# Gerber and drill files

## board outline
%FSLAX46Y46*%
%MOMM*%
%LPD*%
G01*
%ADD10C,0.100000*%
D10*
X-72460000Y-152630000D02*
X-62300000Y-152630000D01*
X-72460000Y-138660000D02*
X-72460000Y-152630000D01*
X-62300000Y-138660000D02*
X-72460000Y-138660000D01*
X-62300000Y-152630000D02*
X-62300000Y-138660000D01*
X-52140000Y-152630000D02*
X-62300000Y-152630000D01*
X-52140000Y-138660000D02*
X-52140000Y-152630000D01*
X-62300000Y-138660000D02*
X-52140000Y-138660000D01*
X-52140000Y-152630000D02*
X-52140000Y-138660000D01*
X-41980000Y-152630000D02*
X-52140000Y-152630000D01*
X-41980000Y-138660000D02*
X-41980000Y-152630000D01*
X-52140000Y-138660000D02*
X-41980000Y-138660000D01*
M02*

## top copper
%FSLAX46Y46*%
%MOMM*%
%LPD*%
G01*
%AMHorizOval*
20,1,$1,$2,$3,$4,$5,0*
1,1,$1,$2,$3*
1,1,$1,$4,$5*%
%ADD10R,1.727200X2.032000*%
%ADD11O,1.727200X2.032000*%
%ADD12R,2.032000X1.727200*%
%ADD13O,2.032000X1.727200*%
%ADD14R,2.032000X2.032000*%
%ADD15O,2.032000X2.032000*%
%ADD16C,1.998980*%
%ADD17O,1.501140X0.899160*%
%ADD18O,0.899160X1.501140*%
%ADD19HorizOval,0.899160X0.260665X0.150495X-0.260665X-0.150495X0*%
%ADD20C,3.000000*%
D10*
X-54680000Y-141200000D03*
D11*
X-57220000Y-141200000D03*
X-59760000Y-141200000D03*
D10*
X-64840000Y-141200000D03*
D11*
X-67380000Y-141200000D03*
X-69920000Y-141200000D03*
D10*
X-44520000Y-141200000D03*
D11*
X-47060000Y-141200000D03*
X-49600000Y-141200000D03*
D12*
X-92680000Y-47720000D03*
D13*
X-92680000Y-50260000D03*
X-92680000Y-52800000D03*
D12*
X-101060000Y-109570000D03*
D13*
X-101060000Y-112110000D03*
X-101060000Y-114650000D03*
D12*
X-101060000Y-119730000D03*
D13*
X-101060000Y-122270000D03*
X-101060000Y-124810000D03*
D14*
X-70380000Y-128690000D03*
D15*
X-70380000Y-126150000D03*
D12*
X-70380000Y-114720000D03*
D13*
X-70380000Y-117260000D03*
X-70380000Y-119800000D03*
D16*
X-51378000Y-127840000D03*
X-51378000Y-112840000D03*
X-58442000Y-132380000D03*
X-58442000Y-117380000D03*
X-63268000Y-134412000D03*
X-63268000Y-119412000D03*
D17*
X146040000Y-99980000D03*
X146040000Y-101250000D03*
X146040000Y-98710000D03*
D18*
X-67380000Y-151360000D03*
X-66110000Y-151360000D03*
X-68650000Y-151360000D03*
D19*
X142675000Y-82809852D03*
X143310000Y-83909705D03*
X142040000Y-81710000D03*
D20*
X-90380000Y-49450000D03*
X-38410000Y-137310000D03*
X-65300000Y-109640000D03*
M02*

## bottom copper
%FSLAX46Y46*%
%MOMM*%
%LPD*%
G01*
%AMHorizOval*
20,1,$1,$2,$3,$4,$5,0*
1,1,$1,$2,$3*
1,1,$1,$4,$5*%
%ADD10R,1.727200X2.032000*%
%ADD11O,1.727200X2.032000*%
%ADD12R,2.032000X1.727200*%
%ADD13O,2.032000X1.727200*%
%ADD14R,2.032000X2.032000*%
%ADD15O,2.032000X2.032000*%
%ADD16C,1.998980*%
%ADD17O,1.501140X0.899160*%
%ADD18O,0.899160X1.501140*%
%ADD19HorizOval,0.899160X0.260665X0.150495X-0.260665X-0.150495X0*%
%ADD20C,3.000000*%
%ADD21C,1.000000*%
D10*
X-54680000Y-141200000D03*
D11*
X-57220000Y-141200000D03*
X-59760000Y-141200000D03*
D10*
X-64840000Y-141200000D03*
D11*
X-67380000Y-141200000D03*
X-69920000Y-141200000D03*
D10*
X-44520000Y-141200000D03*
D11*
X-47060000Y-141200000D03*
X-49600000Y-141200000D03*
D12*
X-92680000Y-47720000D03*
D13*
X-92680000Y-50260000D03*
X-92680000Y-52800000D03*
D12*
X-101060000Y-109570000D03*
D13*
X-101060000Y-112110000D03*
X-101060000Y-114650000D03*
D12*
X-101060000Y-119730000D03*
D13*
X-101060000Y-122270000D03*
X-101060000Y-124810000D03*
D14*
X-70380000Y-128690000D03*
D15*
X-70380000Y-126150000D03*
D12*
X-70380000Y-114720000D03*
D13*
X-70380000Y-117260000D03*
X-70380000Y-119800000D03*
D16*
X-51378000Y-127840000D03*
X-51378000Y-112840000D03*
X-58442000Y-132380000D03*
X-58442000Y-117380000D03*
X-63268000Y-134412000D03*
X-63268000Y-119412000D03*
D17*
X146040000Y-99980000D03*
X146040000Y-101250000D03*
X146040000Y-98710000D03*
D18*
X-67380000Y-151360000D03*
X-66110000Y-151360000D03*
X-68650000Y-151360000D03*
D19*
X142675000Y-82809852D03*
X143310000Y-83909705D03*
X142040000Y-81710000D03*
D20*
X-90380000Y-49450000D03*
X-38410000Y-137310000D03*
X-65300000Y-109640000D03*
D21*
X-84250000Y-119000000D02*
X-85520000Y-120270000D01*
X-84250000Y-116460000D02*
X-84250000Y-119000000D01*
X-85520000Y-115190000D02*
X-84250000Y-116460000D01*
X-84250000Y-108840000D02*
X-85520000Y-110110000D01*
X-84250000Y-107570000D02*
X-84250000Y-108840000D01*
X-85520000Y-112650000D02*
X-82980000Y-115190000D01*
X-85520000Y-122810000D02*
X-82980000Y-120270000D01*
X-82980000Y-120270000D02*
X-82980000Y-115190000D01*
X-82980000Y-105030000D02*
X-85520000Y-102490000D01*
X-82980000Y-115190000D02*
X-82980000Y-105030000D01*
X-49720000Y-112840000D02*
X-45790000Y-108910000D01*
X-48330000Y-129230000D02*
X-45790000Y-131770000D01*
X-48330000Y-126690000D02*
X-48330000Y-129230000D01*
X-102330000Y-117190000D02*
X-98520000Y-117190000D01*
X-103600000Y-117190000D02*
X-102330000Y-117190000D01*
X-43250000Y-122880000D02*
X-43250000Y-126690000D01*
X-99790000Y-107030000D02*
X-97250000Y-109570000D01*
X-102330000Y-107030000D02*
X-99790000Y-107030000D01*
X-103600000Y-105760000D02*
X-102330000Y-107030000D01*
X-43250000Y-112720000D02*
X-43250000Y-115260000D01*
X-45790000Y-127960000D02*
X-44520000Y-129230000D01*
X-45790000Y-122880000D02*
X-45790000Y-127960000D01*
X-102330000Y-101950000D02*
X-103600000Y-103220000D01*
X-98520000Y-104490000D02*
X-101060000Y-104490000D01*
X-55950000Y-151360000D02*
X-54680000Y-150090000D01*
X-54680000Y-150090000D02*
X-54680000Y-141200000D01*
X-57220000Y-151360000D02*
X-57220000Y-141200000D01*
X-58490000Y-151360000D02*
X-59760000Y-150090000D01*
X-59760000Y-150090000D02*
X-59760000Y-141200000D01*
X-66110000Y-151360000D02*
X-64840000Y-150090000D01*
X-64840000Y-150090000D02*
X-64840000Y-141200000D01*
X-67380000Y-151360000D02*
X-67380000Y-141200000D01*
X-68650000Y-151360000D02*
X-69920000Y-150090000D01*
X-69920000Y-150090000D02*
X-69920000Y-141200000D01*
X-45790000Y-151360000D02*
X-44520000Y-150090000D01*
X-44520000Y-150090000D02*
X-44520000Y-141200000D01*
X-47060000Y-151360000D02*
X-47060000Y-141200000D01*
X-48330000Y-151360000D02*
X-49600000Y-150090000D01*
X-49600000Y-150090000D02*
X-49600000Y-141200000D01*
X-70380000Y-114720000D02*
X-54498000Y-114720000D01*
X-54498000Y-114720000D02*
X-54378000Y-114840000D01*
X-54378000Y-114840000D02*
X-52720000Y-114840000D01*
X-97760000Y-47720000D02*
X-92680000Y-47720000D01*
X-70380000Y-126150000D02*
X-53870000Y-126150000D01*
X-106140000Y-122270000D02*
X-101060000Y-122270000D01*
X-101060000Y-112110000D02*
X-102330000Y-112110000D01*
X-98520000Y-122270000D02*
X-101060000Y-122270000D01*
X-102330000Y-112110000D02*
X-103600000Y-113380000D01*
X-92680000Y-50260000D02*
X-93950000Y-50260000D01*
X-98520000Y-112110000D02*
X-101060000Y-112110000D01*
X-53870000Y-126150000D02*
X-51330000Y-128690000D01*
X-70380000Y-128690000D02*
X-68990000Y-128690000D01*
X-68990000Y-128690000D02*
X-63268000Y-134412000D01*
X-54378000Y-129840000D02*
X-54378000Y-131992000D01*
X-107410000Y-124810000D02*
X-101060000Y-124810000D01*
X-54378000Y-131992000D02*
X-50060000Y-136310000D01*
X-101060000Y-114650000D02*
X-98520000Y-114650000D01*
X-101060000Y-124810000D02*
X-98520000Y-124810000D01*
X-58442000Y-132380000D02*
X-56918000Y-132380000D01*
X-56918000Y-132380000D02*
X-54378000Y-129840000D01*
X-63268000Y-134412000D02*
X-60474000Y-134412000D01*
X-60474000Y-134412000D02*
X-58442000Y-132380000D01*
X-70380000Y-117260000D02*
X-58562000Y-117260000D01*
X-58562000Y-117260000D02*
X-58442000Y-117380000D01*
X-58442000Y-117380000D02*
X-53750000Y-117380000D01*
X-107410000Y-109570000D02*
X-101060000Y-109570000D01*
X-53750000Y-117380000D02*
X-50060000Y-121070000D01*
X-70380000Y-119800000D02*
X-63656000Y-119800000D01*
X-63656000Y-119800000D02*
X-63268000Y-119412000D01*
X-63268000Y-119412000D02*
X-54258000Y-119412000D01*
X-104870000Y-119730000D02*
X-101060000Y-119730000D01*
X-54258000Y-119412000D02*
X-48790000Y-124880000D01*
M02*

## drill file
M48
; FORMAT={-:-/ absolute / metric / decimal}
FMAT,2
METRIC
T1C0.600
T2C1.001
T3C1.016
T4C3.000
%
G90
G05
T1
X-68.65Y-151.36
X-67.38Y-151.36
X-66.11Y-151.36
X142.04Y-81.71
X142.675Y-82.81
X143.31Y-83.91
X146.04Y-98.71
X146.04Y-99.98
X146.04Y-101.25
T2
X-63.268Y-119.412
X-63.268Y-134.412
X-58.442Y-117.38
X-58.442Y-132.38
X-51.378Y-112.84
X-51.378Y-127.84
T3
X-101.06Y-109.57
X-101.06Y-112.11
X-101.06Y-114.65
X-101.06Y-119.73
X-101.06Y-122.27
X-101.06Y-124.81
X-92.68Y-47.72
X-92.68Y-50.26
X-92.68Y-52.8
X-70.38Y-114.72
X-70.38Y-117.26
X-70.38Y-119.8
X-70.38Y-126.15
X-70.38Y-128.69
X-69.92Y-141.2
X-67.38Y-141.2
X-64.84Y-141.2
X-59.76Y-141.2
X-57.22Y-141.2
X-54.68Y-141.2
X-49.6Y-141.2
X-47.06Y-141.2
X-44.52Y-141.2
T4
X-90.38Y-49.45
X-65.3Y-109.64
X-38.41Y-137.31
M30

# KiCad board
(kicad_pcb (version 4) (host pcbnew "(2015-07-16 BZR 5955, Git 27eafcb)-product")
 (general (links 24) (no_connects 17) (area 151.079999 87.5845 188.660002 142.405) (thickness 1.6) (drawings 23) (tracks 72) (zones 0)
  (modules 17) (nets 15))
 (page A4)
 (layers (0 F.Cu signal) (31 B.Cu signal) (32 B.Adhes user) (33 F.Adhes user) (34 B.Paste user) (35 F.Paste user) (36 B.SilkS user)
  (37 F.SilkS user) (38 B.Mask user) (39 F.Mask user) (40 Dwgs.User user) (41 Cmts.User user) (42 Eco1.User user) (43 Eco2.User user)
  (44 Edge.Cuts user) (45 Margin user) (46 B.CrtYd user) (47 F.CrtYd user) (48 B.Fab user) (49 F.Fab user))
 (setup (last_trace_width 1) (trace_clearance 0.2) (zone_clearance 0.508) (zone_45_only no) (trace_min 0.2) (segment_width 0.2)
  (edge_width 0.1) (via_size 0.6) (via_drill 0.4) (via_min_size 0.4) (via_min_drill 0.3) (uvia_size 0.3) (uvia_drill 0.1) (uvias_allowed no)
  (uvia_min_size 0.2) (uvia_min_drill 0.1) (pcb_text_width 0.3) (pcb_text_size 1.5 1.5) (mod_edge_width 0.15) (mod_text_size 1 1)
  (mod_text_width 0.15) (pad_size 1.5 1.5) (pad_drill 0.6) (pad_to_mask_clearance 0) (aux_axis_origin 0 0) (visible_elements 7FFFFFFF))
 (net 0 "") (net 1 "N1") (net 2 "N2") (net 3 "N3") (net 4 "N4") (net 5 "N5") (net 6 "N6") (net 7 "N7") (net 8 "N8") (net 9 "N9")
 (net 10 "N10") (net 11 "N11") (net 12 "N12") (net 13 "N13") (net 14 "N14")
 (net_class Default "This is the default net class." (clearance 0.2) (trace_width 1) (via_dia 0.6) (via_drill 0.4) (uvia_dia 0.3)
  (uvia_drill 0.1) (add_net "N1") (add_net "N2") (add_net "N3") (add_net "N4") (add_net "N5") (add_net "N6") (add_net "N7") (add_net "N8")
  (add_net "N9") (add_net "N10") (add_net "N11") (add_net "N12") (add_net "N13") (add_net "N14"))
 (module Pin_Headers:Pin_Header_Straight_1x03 (layer F.Cu) (at -54.68 141.2 270)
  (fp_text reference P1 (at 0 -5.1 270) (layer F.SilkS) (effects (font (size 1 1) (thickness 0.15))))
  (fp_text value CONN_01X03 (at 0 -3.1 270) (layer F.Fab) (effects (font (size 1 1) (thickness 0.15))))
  (pad 1 thru_hole rect (at 0 0 270) (size 2.032 1.7272) (drill 1.016) (layers *.Cu *.Mask F.SilkS) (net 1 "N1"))
  (pad 2 thru_hole oval (at 0 2.54 270) (size 2.032 1.7272) (drill 1.016) (layers *.Cu *.Mask F.SilkS) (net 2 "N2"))
  (pad 3 thru_hole oval (at 0 5.08 270) (size 2.032 1.7272) (drill 1.016) (layers *.Cu *.Mask F.SilkS) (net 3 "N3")))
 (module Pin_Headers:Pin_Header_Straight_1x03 (layer F.Cu) (at -64.84 141.2 270)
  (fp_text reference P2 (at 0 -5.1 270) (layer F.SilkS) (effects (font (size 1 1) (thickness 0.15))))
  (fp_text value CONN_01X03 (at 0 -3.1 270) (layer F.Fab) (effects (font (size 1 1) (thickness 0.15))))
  (pad 1 thru_hole rect (at 0 0 270) (size 2.032 1.7272) (drill 1.016) (layers *.Cu *.Mask F.SilkS) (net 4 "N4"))
  (pad 2 thru_hole oval (at 0 2.54 270) (size 2.032 1.7272) (drill 1.016) (layers *.Cu *.Mask F.SilkS) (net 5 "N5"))
  (pad 3 thru_hole oval (at 0 5.08 270) (size 2.032 1.7272) (drill 1.016) (layers *.Cu *.Mask F.SilkS) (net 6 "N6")))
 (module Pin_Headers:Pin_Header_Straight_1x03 (layer F.Cu) (at -44.52 141.2 270)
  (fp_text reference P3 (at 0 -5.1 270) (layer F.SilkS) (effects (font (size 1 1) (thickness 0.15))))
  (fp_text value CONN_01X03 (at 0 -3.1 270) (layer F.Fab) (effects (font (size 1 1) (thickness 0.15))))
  (pad 1 thru_hole rect (at 0 0 270) (size 2.032 1.7272) (drill 1.016) (layers *.Cu *.Mask F.SilkS) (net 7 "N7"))
  (pad 2 thru_hole oval (at 0 2.54 270) (size 2.032 1.7272) (drill 1.016) (layers *.Cu *.Mask F.SilkS) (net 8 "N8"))
  (pad 3 thru_hole oval (at 0 5.08 270) (size 2.032 1.7272) (drill 1.016) (layers *.Cu *.Mask F.SilkS) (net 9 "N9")))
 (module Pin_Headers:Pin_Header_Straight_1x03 (layer F.Cu) (at -92.68 47.72)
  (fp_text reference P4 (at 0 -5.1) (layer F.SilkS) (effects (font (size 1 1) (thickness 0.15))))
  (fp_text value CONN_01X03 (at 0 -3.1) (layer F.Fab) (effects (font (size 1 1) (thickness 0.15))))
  (pad 1 thru_hole rect (at 0 0) (size 2.032 1.7272) (drill 1.016) (layers *.Cu *.Mask F.SilkS) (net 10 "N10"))
  (pad 2 thru_hole oval (at 0 2.54) (size 2.032 1.7272) (drill 1.016) (layers *.Cu *.Mask F.SilkS) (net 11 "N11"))
  (pad 3 thru_hole oval (at 0 5.08) (size 2.032 1.7272) (drill 1.016) (layers *.Cu *.Mask F.SilkS) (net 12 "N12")))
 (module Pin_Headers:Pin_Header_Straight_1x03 (layer F.Cu) (at -101.06 109.57)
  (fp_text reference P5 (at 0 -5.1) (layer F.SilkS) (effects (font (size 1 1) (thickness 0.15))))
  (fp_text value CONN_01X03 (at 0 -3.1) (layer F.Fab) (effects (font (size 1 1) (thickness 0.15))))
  (pad 1 thru_hole rect (at 0 0) (size 2.032 1.7272) (drill 1.016) (layers *.Cu *.Mask F.SilkS) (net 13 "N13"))
  (pad 2 thru_hole oval (at 0 2.54) (size 2.032 1.7272) (drill 1.016) (layers *.Cu *.Mask F.SilkS) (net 11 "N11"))
  (pad 3 thru_hole oval (at 0 5.08) (size 2.032 1.7272) (drill 1.016) (layers *.Cu *.Mask F.SilkS) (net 12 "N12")))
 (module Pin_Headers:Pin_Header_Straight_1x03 (layer F.Cu) (at -101.06 119.73)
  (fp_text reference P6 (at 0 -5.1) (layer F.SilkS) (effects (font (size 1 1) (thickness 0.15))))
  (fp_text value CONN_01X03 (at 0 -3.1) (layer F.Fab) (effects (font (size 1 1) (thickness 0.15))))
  (pad 1 thru_hole rect (at 0 0) (size 2.032 1.7272) (drill 1.016) (layers *.Cu *.Mask F.SilkS) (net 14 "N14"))
  (pad 2 thru_hole oval (at 0 2.54) (size 2.032 1.7272) (drill 1.016) (layers *.Cu *.Mask F.SilkS) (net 11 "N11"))
  (pad 3 thru_hole oval (at 0 5.08) (size 2.032 1.7272) (drill 1.016) (layers *.Cu *.Mask F.SilkS) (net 12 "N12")))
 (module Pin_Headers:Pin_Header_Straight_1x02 (layer F.Cu) (at -70.38 128.69 180)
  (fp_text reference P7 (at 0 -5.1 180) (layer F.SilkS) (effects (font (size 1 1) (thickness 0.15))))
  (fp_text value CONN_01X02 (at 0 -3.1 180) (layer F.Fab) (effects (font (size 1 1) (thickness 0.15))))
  (pad 1 thru_hole rect (at 0 0 180) (size 2.032 2.032) (drill 1.016) (layers *.Cu *.Mask F.SilkS) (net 12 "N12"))
  (pad 2 thru_hole oval (at 0 2.54 180) (size 2.032 2.032) (drill 1.016) (layers *.Cu *.Mask F.SilkS) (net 11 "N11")))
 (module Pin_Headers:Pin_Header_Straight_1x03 (layer F.Cu) (at -70.38 114.72)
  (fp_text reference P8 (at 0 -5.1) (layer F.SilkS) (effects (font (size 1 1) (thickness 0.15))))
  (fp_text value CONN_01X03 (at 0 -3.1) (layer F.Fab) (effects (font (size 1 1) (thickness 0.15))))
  (pad 1 thru_hole rect (at 0 0) (size 2.032 1.7272) (drill 1.016) (layers *.Cu *.Mask F.SilkS) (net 10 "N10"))
  (pad 2 thru_hole oval (at 0 2.54) (size 2.032 1.7272) (drill 1.016) (layers *.Cu *.Mask F.SilkS) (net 13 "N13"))
  (pad 3 thru_hole oval (at 0 5.08) (size 2.032 1.7272) (drill 1.016) (layers *.Cu *.Mask F.SilkS) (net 14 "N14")))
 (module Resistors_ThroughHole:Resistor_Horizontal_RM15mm (layer F.Cu) (at -51.378 120.34 90)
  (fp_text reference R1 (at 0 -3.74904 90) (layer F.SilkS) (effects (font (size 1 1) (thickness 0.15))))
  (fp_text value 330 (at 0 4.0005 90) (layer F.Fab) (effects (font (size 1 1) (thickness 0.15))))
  (pad 1 thru_hole circle (at -7.5 0 90) (size 1.99898 1.99898) (drill 1.00076) (layers *.Cu *.SilkS *.Mask) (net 12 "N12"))
  (pad 2 thru_hole circle (at 7.5 0 90) (size 1.99898 1.99898) (drill 1.00076) (layers *.Cu *.SilkS *.Mask) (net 10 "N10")))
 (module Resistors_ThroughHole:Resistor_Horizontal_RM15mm (layer F.Cu) (at -58.442 124.88 90)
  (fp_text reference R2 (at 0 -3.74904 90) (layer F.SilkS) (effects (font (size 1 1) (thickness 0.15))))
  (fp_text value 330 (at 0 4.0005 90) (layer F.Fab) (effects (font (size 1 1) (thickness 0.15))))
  (pad 1 thru_hole circle (at -7.5 0 90) (size 1.99898 1.99898) (drill 1.00076) (layers *.Cu *.SilkS *.Mask) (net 12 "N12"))
  (pad 2 thru_hole circle (at 7.5 0 90) (size 1.99898 1.99898) (drill 1.00076) (layers *.Cu *.SilkS *.Mask) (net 13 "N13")))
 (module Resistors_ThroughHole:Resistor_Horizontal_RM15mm (layer F.Cu) (at -63.268 126.912 90)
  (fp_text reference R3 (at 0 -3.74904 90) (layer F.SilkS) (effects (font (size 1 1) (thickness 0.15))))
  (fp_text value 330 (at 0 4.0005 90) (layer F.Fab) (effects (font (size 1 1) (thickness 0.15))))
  (pad 1 thru_hole circle (at -7.5 0 90) (size 1.99898 1.99898) (drill 1.00076) (layers *.Cu *.SilkS *.Mask) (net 12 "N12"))
  (pad 2 thru_hole circle (at 7.5 0 90) (size 1.99898 1.99898) (drill 1.00076) (layers *.Cu *.SilkS *.Mask) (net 14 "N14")))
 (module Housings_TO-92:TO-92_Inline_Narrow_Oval (layer F.Cu) (at 146.04 98.71 270)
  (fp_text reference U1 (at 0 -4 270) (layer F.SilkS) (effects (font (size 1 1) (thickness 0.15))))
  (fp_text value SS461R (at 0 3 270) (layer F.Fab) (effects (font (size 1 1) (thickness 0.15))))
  (pad 2 thru_hole oval (at 1.27 0 90) (size 0.89916 1.50114) (drill 0.6) (layers *.Cu *.Mask F.SilkS) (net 2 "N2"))
  (pad 3 thru_hole oval (at 2.54 0 90) (size 0.89916 1.50114) (drill 0.6) (layers *.Cu *.Mask F.SilkS) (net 1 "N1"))
  (pad 1 thru_hole oval (at 0 0 90) (size 0.89916 1.50114) (drill 0.6) (layers *.Cu *.Mask F.SilkS) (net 3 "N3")))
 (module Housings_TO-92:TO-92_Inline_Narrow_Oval (layer F.Cu) (at -68.65 151.36)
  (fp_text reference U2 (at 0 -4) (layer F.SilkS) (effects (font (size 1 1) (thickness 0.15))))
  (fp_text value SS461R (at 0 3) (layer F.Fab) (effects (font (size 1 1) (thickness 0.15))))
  (pad 2 thru_hole oval (at 1.27 0 180) (size 0.89916 1.50114) (drill 0.6) (layers *.Cu *.Mask F.SilkS) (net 5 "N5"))
  (pad 3 thru_hole oval (at 2.54 0 180) (size 0.89916 1.50114) (drill 0.6) (layers *.Cu *.Mask F.SilkS) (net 4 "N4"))
  (pad 1 thru_hole oval (at 0 0 180) (size 0.89916 1.50114) (drill 0.6) (layers *.Cu *.Mask F.SilkS) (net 6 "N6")))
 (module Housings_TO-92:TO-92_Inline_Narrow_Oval (layer F.Cu) (at 142.04 81.71 300)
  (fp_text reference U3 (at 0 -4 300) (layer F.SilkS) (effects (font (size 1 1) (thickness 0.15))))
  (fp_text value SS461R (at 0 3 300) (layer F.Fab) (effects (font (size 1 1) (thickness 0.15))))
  (pad 2 thru_hole oval (at 1.27 0 120) (size 0.89916 1.50114) (drill 0.6) (layers *.Cu *.Mask F.SilkS) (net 8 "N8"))
  (pad 3 thru_hole oval (at 2.54 0 120) (size 0.89916 1.50114) (drill 0.6) (layers *.Cu *.Mask F.SilkS) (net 7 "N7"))
  (pad 1 thru_hole oval (at 0 0 120) (size 0.89916 1.50114) (drill 0.6) (layers *.Cu *.Mask F.SilkS) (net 9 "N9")))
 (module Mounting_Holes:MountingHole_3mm (layer F.Cu) (at -90.38 49.45)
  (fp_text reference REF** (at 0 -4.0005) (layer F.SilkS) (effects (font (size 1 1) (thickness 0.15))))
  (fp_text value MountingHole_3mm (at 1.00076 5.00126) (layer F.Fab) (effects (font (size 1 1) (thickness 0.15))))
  (pad 1 thru_hole circle (at 0 0) (size 3 3) (drill 3) (layers)))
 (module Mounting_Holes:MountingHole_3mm (layer F.Cu) (at -38.41 137.31)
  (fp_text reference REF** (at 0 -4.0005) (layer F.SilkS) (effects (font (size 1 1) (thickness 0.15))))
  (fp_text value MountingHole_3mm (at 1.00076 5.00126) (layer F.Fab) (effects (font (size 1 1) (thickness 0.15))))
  (pad 1 thru_hole circle (at 0 0) (size 3 3) (drill 3) (layers)))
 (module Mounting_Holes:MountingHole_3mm (layer F.Cu) (at -65.3 109.64)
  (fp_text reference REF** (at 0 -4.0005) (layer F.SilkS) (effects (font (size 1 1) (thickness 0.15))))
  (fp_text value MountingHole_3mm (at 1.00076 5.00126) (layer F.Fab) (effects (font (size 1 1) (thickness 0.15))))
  (pad 1 thru_hole circle (at 0 0) (size 3 3) (drill 3) (layers)))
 (gr_line (start -72.46 152.63) (end -62.3 152.63) (angle 90) (layer Edge.Cuts) (width 0.1))
 (gr_line (start -72.46 138.66) (end -72.46 152.63) (angle 90) (layer Edge.Cuts) (width 0.1))
 (gr_line (start -62.3 138.66) (end -72.46 138.66) (angle 90) (layer Edge.Cuts) (width 0.1))
 (gr_line (start -62.3 152.63) (end -62.3 138.66) (angle 90) (layer Edge.Cuts) (width 0.1))
 (gr_line (start -52.14 152.63) (end -62.3 152.63) (angle 90) (layer Edge.Cuts) (width 0.1))
 (gr_line (start -52.14 138.66) (end -52.14 152.63) (angle 90) (layer Edge.Cuts) (width 0.1))
 (gr_line (start -62.3 138.66) (end -52.14 138.66) (angle 90) (layer Edge.Cuts) (width 0.1))
 (gr_line (start -52.14 152.63) (end -52.14 138.66) (angle 90) (layer Edge.Cuts) (width 0.1))
 (gr_line (start -41.98 152.63) (end -52.14 152.63) (angle 90) (layer Edge.Cuts) (width 0.1))
 (gr_line (start -41.98 138.66) (end -41.98 152.63) (angle 90) (layer Edge.Cuts) (width 0.1))
 (gr_line (start -52.14 138.66) (end -41.98 138.66) (angle 90) (layer Edge.Cuts) (width 0.1))
 (segment (start -84.25 119) (end -85.52 120.27) (width 1) (layer B.Cu) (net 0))
 (segment (start -84.25 116.46) (end -84.25 119) (width 1) (layer B.Cu) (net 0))
 (segment (start -85.52 115.19) (end -84.25 116.46) (width 1) (layer B.Cu) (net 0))
 (segment (start -84.25 108.84) (end -85.52 110.11) (width 1) (layer B.Cu) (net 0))
 (segment (start -84.25 107.57) (end -84.25 108.84) (width 1) (layer B.Cu) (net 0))
 (segment (start -85.52 112.65) (end -82.98 115.19) (width 1) (layer B.Cu) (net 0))
 (segment (start -85.52 122.81) (end -82.98 120.27) (width 1) (layer B.Cu) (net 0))
 (segment (start -82.98 120.27) (end -82.98 115.19) (width 1) (layer B.Cu) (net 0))
 (segment (start -82.98 105.03) (end -85.52 102.49) (width 1) (layer B.Cu) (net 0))
 (segment (start -82.98 115.19) (end -82.98 105.03) (width 1) (layer B.Cu) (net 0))
 (segment (start -49.72 112.84) (end -45.79 108.91) (width 1) (layer B.Cu) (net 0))
 (segment (start -48.33 129.23) (end -45.79 131.77) (width 1) (layer B.Cu) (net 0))
 (segment (start -48.33 126.69) (end -48.33 129.23) (width 1) (layer B.Cu) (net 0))
 (segment (start -102.33 117.19) (end -98.52 117.19) (width 1) (layer B.Cu) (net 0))
 (segment (start -103.6 117.19) (end -102.33 117.19) (width 1) (layer B.Cu) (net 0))
 (segment (start -43.25 122.88) (end -43.25 126.69) (width 1) (layer B.Cu) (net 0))
 (segment (start -99.79 107.03) (end -97.25 109.57) (width 1) (layer B.Cu) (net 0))
 (segment (start -102.33 107.03) (end -99.79 107.03) (width 1) (layer B.Cu) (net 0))
 (segment (start -103.6 105.76) (end -102.33 107.03) (width 1) (layer B.Cu) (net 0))
 (segment (start -43.25 112.72) (end -43.25 115.26) (width 1) (layer B.Cu) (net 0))
 (segment (start -45.79 127.96) (end -44.52 129.23) (width 1) (layer B.Cu) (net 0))
 (segment (start -45.79 122.88) (end -45.79 127.96) (width 1) (layer B.Cu) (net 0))
 (segment (start -102.33 101.95) (end -103.6 103.22) (width 1) (layer B.Cu) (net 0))
 (segment (start -98.52 104.49) (end -101.06 104.49) (width 1) (layer B.Cu) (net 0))
 (segment (start -55.95 151.36) (end -54.68 150.09) (width 1) (layer B.Cu) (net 1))
 (segment (start -54.68 150.09) (end -54.68 141.2) (width 1) (layer B.Cu) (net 1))
 (segment (start -57.22 151.36) (end -57.22 141.2) (width 1) (layer B.Cu) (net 2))
 (segment (start -58.49 151.36) (end -59.76 150.09) (width 1) (layer B.Cu) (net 3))
 (segment (start -59.76 150.09) (end -59.76 141.2) (width 1) (layer B.Cu) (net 3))
 (segment (start -66.11 151.36) (end -64.84 150.09) (width 1) (layer B.Cu) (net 4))
 (segment (start -64.84 150.09) (end -64.84 141.2) (width 1) (layer B.Cu) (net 4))
 (segment (start -67.38 151.36) (end -67.38 141.2) (width 1) (layer B.Cu) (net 5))
 (segment (start -68.65 151.36) (end -69.92 150.09) (width 1) (layer B.Cu) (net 6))
 (segment (start -69.92 150.09) (end -69.92 141.2) (width 1) (layer B.Cu) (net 6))
 (segment (start -45.79 151.36) (end -44.52 150.09) (width 1) (layer B.Cu) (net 7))
 (segment (start -44.52 150.09) (end -44.52 141.2) (width 1) (layer B.Cu) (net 7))
 (segment (start -47.06 151.36) (end -47.06 141.2) (width 1) (layer B.Cu) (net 8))
 (segment (start -48.33 151.36) (end -49.6 150.09) (width 1) (layer B.Cu) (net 9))
 (segment (start -49.6 150.09) (end -49.6 141.2) (width 1) (layer B.Cu) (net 9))
 (segment (start -70.38 114.72) (end -54.498 114.72) (width 1) (layer B.Cu) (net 10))
 (segment (start -54.498 114.72) (end -54.378 114.84) (width 1) (layer B.Cu) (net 10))
 (segment (start -54.378 114.84) (end -52.72 114.84) (width 1) (layer B.Cu) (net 10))
 (segment (start -97.76 47.72) (end -92.68 47.72) (width 1) (layer B.Cu) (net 10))
 (segment (start -70.38 126.15) (end -53.87 126.15) (width 1) (layer B.Cu) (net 11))
 (segment (start -106.14 122.27) (end -101.06 122.27) (width 1) (layer B.Cu) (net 11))
 (segment (start -101.06 112.11) (end -102.33 112.11) (width 1) (layer B.Cu) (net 11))
 (segment (start -98.52 122.27) (end -101.06 122.27) (width 1) (layer B.Cu) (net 11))
 (segment (start -102.33 112.11) (end -103.6 113.38) (width 1) (layer B.Cu) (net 11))
 (segment (start -92.68 50.26) (end -93.95 50.26) (width 1) (layer B.Cu) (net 11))
 (segment (start -98.52 112.11) (end -101.06 112.11) (width 1) (layer B.Cu) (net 11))
 (segment (start -53.87 126.15) (end -51.33 128.69) (width 1) (layer B.Cu) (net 12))
 (segment (start -70.38 128.69) (end -68.99 128.69) (width 1) (layer B.Cu) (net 12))
 (segment (start -68.99 128.69) (end -63.268 134.412) (width 1) (layer B.Cu) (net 12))
 (segment (start -54.378 129.84) (end -54.378 131.992) (width 1) (layer B.Cu) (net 12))
 (segment (start -107.41 124.81) (end -101.06 124.81) (width 1) (layer B.Cu) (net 12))
 (segment (start -54.378 131.992) (end -50.06 136.31) (width 1) (layer B.Cu) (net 12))
 (segment (start -101.06 114.65) (end -98.52 114.65) (width 1) (layer B.Cu) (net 12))
 (segment (start -101.06 124.81) (end -98.52 124.81) (width 1) (layer B.Cu) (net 12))
 (segment (start -58.442 132.38) (end -56.918 132.38) (width 1) (layer B.Cu) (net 12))
 (segment (start -56.918 132.38) (end -54.378 129.84) (width 1) (layer B.Cu) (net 12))
 (segment (start -63.268 134.412) (end -60.474 134.412) (width 1) (layer B.Cu) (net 12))
 (segment (start -60.474 134.412) (end -58.442 132.38) (width 1) (layer B.Cu) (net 12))
 (segment (start -70.38 117.26) (end -58.562 117.26) (width 1) (layer B.Cu) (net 13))
 (segment (start -58.562 117.26) (end -58.442 117.38) (width 1) (layer B.Cu) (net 13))
 (segment (start -58.442 117.38) (end -53.75 117.38) (width 1) (layer B.Cu) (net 13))
 (segment (start -107.41 109.57) (end -101.06 109.57) (width 1) (layer B.Cu) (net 13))
 (segment (start -53.75 117.38) (end -50.06 121.07) (width 1) (layer B.Cu) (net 13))
 (segment (start -70.38 119.8) (end -63.656 119.8) (width 1) (layer B.Cu) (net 14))
 (segment (start -63.656 119.8) (end -63.268 119.412) (width 1) (layer B.Cu) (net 14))
 (segment (start -63.268 119.412) (end -54.258 119.412) (width 1) (layer B.Cu) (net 14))
 (segment (start -104.87 119.73) (end -101.06 119.73) (width 1) (layer B.Cu) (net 14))
 (segment (start -54.258 119.412) (end -48.79 124.88) (width 1) (layer B.Cu) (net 14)))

